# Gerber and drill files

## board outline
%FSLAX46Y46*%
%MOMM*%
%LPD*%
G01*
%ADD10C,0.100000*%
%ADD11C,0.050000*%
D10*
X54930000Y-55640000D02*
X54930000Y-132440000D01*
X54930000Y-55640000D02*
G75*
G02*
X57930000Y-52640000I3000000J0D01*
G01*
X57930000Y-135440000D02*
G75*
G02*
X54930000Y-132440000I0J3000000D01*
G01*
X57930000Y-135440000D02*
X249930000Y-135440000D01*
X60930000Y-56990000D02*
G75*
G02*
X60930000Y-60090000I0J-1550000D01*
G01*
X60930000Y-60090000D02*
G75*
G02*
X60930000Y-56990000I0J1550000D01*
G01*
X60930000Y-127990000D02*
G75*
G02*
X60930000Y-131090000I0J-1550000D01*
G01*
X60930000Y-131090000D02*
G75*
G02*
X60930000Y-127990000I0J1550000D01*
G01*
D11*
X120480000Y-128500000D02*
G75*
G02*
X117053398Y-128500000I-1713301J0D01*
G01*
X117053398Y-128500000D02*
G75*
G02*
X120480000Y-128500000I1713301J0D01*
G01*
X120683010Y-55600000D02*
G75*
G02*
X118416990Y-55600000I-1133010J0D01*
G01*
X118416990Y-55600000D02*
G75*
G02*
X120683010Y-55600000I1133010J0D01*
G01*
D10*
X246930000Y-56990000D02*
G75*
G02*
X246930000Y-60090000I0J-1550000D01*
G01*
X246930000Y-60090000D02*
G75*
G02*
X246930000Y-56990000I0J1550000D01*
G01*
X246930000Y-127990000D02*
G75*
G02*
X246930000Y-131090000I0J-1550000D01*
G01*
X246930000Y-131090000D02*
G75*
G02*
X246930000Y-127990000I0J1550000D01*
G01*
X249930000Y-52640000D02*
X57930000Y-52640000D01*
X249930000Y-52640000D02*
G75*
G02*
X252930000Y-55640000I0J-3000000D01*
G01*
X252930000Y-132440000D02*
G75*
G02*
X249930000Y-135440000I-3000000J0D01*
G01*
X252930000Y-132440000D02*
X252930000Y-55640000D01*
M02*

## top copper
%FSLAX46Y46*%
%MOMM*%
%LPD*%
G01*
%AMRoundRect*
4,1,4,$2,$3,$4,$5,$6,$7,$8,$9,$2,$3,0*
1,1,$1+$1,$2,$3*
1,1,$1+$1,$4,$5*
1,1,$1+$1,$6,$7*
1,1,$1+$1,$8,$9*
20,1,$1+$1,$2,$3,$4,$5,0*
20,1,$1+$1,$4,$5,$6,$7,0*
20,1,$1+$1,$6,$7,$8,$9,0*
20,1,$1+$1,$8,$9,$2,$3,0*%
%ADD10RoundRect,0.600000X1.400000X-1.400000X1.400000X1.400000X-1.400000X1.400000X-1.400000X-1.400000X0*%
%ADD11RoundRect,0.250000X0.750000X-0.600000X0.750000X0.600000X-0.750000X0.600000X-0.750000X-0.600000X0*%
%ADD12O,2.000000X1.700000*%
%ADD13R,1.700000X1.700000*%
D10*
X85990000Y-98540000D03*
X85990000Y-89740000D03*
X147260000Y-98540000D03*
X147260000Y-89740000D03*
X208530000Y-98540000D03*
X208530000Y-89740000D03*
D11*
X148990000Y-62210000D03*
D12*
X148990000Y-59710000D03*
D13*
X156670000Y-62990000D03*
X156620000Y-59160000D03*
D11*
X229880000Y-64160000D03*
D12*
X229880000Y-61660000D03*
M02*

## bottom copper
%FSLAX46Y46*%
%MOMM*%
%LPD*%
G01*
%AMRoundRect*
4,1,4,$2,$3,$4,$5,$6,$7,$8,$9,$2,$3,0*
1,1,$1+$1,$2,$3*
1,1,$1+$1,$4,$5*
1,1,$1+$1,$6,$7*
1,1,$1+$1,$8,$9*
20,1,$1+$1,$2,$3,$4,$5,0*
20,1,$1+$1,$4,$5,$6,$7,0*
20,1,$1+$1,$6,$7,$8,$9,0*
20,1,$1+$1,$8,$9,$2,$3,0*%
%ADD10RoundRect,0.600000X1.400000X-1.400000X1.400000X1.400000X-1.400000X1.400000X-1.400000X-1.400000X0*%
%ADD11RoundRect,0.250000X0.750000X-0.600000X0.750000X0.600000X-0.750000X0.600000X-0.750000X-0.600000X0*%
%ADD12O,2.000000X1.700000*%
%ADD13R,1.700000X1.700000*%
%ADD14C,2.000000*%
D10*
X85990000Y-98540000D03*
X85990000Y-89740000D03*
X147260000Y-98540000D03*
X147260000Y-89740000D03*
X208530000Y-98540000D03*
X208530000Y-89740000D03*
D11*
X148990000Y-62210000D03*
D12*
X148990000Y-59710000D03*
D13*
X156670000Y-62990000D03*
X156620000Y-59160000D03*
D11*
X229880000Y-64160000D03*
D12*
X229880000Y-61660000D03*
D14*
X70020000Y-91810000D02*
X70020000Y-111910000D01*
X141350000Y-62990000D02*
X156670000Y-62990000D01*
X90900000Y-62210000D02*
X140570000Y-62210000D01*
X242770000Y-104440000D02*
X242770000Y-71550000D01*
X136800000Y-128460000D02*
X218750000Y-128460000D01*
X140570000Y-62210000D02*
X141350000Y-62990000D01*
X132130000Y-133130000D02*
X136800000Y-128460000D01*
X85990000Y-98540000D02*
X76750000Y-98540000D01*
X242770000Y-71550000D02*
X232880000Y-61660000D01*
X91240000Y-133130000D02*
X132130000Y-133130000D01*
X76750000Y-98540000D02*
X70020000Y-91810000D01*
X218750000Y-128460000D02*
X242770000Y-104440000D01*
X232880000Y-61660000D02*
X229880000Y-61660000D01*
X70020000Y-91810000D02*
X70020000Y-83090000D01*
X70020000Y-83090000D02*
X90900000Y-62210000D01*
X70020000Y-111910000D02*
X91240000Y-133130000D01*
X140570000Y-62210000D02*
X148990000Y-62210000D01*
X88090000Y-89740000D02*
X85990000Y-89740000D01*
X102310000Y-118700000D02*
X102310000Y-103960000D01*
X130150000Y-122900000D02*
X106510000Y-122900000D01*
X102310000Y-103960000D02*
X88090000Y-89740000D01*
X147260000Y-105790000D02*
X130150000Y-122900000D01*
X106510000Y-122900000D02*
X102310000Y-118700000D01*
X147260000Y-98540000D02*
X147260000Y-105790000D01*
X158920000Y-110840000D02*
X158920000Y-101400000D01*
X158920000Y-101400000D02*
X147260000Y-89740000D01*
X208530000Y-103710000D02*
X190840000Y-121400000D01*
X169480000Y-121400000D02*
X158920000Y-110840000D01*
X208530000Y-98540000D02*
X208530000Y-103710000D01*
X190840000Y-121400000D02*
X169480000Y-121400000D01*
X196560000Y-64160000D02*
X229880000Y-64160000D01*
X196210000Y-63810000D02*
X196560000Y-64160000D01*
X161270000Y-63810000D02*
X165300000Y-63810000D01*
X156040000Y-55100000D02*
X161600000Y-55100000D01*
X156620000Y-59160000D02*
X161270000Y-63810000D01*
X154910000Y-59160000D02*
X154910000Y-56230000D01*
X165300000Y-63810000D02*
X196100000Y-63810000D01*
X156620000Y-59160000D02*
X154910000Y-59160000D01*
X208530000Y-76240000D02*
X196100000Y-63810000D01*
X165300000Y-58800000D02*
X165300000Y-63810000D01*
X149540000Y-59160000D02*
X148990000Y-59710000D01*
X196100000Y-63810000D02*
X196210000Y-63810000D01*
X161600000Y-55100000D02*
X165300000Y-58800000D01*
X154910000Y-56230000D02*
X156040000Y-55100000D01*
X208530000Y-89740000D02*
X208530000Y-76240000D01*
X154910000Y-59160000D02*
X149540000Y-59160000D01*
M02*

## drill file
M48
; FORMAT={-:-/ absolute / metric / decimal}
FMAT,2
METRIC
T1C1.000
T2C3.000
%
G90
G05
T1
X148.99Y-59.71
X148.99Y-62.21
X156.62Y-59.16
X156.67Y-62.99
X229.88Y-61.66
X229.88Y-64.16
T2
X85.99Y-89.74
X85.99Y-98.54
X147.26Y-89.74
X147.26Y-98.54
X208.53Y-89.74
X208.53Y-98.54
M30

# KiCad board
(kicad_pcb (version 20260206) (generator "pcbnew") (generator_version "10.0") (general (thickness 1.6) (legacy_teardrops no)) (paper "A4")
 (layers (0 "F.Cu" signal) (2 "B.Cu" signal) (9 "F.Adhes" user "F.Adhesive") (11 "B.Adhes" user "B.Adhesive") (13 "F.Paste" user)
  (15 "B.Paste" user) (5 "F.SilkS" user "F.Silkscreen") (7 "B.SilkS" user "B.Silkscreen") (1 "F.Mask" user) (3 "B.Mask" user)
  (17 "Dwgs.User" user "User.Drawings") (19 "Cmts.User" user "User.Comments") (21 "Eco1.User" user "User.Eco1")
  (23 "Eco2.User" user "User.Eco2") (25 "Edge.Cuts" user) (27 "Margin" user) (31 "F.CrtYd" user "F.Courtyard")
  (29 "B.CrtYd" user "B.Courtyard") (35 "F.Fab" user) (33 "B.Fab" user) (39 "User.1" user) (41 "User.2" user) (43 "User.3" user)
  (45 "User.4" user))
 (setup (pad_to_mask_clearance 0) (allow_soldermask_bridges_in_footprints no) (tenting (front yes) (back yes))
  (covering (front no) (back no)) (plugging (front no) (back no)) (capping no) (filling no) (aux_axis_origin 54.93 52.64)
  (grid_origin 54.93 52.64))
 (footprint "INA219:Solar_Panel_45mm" (layer "F.Cu") (at 85.99 94.14 90)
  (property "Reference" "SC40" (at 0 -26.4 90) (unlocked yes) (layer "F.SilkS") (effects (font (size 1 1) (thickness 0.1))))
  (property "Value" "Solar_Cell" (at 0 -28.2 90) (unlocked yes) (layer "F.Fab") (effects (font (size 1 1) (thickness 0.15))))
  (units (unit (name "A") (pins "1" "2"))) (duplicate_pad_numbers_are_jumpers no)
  (pad "1" thru_hole roundrect (at -4.4 0 90) (size 4 4) (drill 3) (layers "*.Cu" "*.Mask") (remove_unused_layers no)
   (roundrect_rratio 0.15) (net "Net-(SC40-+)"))
  (pad "2" thru_hole roundrect (at 4.4 0 90) (size 4 4) (drill 3) (layers "*.Cu" "*.Mask") (remove_unused_layers no) (roundrect_rratio 0.15)
   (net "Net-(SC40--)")))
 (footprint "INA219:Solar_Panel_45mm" (layer "F.Cu") (at 147.26 94.14 90)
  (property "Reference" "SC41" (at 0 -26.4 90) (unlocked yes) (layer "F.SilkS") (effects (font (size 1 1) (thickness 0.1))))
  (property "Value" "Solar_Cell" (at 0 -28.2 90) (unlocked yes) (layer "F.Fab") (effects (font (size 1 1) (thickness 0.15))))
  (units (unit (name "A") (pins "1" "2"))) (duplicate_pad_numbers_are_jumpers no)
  (pad "1" thru_hole roundrect (at -4.4 0 90) (size 4 4) (drill 3) (layers "*.Cu" "*.Mask") (remove_unused_layers no)
   (roundrect_rratio 0.15) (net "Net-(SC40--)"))
  (pad "2" thru_hole roundrect (at 4.4 0 90) (size 4 4) (drill 3) (layers "*.Cu" "*.Mask") (remove_unused_layers no) (roundrect_rratio 0.15)
   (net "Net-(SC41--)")))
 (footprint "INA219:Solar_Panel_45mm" (layer "F.Cu") (at 208.53 94.14 90)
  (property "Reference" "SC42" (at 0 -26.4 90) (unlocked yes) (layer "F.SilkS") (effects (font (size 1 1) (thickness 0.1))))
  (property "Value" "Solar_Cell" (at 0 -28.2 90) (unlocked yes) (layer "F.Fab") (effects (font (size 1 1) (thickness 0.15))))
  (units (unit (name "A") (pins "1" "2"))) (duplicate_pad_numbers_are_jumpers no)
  (pad "1" thru_hole roundrect (at -4.4 0 90) (size 4 4) (drill 3) (layers "*.Cu" "*.Mask") (remove_unused_layers no)
   (roundrect_rratio 0.15) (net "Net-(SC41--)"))
  (pad "2" thru_hole roundrect (at 4.4 0 90) (size 4 4) (drill 3) (layers "*.Cu" "*.Mask") (remove_unused_layers no) (roundrect_rratio 0.15)
   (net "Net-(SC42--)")))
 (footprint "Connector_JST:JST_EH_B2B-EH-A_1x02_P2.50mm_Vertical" (layer "B.Cu") (at 148.99 62.21 90)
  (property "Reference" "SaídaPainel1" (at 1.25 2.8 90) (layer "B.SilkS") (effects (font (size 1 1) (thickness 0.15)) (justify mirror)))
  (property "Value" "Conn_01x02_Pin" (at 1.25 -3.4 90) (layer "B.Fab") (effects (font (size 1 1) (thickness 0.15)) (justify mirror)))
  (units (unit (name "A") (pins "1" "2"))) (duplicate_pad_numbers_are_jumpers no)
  (pad "1" thru_hole roundrect (at 0 0 90) (size 1.7 2) (drill 1) (layers "*.Cu" "*.Mask") (remove_unused_layers no)
   (roundrect_rratio 0.147059) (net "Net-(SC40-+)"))
  (pad "2" thru_hole oval (at 2.5 0 90) (size 1.7 2) (drill 1) (layers "*.Cu" "*.Mask") (remove_unused_layers no) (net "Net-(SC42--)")))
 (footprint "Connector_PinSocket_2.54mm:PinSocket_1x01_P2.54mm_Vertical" (layer "B.Cu") (at 156.67 62.99 90)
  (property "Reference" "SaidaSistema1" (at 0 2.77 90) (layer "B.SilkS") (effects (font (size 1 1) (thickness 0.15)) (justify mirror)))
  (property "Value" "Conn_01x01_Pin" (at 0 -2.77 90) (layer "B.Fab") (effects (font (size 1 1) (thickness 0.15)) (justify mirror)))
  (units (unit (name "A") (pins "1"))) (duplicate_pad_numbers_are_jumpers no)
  (pad "1" thru_hole rect (at 0 0 90) (size 1.7 1.7) (drill 1) (layers "*.Cu" "*.Mask") (remove_unused_layers no) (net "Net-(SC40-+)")))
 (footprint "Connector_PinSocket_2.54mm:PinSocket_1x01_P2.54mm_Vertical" (layer "B.Cu") (at 156.62 59.16 90)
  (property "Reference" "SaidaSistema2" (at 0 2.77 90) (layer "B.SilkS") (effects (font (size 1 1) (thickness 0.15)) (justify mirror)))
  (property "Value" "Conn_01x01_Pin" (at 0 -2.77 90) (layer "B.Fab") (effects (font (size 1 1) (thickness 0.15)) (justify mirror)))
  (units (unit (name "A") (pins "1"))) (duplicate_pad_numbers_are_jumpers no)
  (pad "1" thru_hole rect (at 0 0 90) (size 1.7 1.7) (drill 1) (layers "*.Cu" "*.Mask") (remove_unused_layers no) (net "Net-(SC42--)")))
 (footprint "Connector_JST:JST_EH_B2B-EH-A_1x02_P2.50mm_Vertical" (layer "B.Cu") (at 229.88 64.16 90)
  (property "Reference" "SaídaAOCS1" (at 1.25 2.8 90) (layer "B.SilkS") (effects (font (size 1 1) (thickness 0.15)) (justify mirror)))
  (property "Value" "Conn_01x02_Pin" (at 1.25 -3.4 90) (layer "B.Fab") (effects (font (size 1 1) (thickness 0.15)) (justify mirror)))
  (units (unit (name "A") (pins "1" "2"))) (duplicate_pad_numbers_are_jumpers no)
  (pad "1" thru_hole roundrect (at 0 0 90) (size 1.7 2) (drill 1) (layers "*.Cu" "*.Mask") (remove_unused_layers no)
   (roundrect_rratio 0.147059) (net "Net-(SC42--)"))
  (pad "2" thru_hole oval (at 2.5 0 90) (size 1.7 2) (drill 1) (layers "*.Cu" "*.Mask") (remove_unused_layers no) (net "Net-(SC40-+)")))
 (gr_line (start 54.93 55.64) (end 54.93 132.44) (stroke (width 0.1) (type default)) (layer "Edge.Cuts"))
 (gr_arc (start 54.93 55.64) (mid 55.80868 53.51868) (end 57.93 52.64) (stroke (width 0.1) (type default)) (layer "Edge.Cuts"))
 (gr_arc (start 57.93 135.44) (mid 55.80868 134.56132) (end 54.93 132.44) (stroke (width 0.1) (type default)) (layer "Edge.Cuts"))
 (gr_line (start 57.93 135.44) (end 249.93 135.44) (stroke (width 0.1) (type default)) (layer "Edge.Cuts"))
 (gr_arc (start 60.93 56.99) (mid 62.48 58.54) (end 60.93 60.09) (stroke (width 0.1) (type default)) (layer "Edge.Cuts"))
 (gr_arc (start 60.93 60.09) (mid 59.38 58.54) (end 60.93 56.99) (stroke (width 0.1) (type default)) (layer "Edge.Cuts"))
 (gr_arc (start 60.93 127.99) (mid 62.48 129.54) (end 60.93 131.09) (stroke (width 0.1) (type default)) (layer "Edge.Cuts"))
 (gr_arc (start 60.93 131.09) (mid 59.38 129.54) (end 60.93 127.99) (stroke (width 0.1) (type default)) (layer "Edge.Cuts"))
 (gr_circle (center 118.766699 128.5) (end 120.316699 127.77) (stroke (width 0.05) (type default)) (fill no) (layer "Edge.Cuts"))
 (gr_circle (center 119.55 55.6) (end 120.68301 55.6) (stroke (width 0.05) (type solid)) (fill no) (layer "Edge.Cuts"))
 (gr_arc (start 246.93 56.99) (mid 248.48 58.54) (end 246.93 60.09) (stroke (width 0.1) (type default)) (layer "Edge.Cuts"))
 (gr_arc (start 246.93 60.09) (mid 245.38 58.54) (end 246.93 56.99) (stroke (width 0.1) (type default)) (layer "Edge.Cuts"))
 (gr_arc (start 246.93 127.99) (mid 248.48 129.54) (end 246.93 131.09) (stroke (width 0.1) (type default)) (layer "Edge.Cuts"))
 (gr_arc (start 246.93 131.09) (mid 245.38 129.54) (end 246.93 127.99) (stroke (width 0.1) (type default)) (layer "Edge.Cuts"))
 (gr_line (start 249.93 52.64) (end 57.93 52.64) (stroke (width 0.1) (type default)) (layer "Edge.Cuts"))
 (gr_arc (start 249.93 52.64) (mid 252.05132 53.51868) (end 252.93 55.64) (stroke (width 0.1) (type default)) (layer "Edge.Cuts"))
 (gr_arc (start 252.93 132.44) (mid 252.05132 134.56132) (end 249.93 135.44) (stroke (width 0.1) (type default)) (layer "Edge.Cuts"))
 (gr_line (start 252.93 132.44) (end 252.93 55.64) (stroke (width 0.1) (type default)) (layer "Edge.Cuts"))
 (segment (start 70.02 91.81) (end 70.02 111.91) (width 2) (layer "B.Cu") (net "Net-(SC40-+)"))
 (segment (start 141.35 62.99) (end 156.67 62.99) (width 2) (layer "B.Cu") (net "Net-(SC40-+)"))
 (segment (start 90.9 62.21) (end 140.57 62.21) (width 2) (layer "B.Cu") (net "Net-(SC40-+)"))
 (segment (start 242.77 104.44) (end 242.77 71.55) (width 2) (layer "B.Cu") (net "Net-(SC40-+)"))
 (segment (start 136.8 128.46) (end 218.75 128.46) (width 2) (layer "B.Cu") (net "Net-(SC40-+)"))
 (segment (start 140.57 62.21) (end 141.35 62.99) (width 2) (layer "B.Cu") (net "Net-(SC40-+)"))
 (segment (start 132.13 133.13) (end 136.8 128.46) (width 2) (layer "B.Cu") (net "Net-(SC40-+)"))
 (segment (start 85.99 98.54) (end 76.75 98.54) (width 2) (layer "B.Cu") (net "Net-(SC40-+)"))
 (segment (start 242.77 71.55) (end 232.88 61.66) (width 2) (layer "B.Cu") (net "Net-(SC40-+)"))
 (segment (start 91.24 133.13) (end 132.13 133.13) (width 2) (layer "B.Cu") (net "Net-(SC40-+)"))
 (segment (start 76.75 98.54) (end 70.02 91.81) (width 2) (layer "B.Cu") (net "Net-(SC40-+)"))
 (segment (start 218.75 128.46) (end 242.77 104.44) (width 2) (layer "B.Cu") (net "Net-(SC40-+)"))
 (segment (start 232.88 61.66) (end 229.88 61.66) (width 2) (layer "B.Cu") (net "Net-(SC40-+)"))
 (segment (start 70.02 91.81) (end 70.02 83.09) (width 2) (layer "B.Cu") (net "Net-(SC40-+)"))
 (segment (start 70.02 83.09) (end 90.9 62.21) (width 2) (layer "B.Cu") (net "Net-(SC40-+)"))
 (segment (start 70.02 111.91) (end 91.24 133.13) (width 2) (layer "B.Cu") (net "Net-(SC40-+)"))
 (segment (start 140.57 62.21) (end 148.99 62.21) (width 2) (layer "B.Cu") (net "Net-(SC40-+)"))
 (segment (start 88.09 89.74) (end 85.99 89.74) (width 2) (layer "B.Cu") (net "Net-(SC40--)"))
 (segment (start 102.31 118.7) (end 102.31 103.96) (width 2) (layer "B.Cu") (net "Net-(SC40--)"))
 (segment (start 130.15 122.9) (end 106.51 122.9) (width 2) (layer "B.Cu") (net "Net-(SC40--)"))
 (segment (start 102.31 103.96) (end 88.09 89.74) (width 2) (layer "B.Cu") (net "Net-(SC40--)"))
 (segment (start 147.26 105.79) (end 130.15 122.9) (width 2) (layer "B.Cu") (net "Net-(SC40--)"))
 (segment (start 106.51 122.9) (end 102.31 118.7) (width 2) (layer "B.Cu") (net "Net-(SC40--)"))
 (segment (start 147.26 98.54) (end 147.26 105.79) (width 2) (layer "B.Cu") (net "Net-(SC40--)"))
 (segment (start 158.92 110.84) (end 158.92 101.4) (width 2) (layer "B.Cu") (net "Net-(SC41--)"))
 (segment (start 158.92 101.4) (end 147.26 89.74) (width 2) (layer "B.Cu") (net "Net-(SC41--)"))
 (segment (start 208.53 103.71) (end 190.84 121.4) (width 2) (layer "B.Cu") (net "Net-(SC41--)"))
 (segment (start 169.48 121.4) (end 158.92 110.84) (width 2) (layer "B.Cu") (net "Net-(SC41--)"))
 (segment (start 208.53 98.54) (end 208.53 103.71) (width 2) (layer "B.Cu") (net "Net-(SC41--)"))
 (segment (start 190.84 121.4) (end 169.48 121.4) (width 2) (layer "B.Cu") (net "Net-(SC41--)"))
 (segment (start 196.56 64.16) (end 229.88 64.16) (width 2) (layer "B.Cu") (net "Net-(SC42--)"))
 (segment (start 196.21 63.81) (end 196.56 64.16) (width 2) (layer "B.Cu") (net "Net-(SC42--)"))
 (segment (start 161.27 63.81) (end 165.3 63.81) (width 2) (layer "B.Cu") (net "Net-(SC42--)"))
 (segment (start 156.04 55.1) (end 161.6 55.1) (width 2) (layer "B.Cu") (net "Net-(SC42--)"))
 (segment (start 156.62 59.16) (end 161.27 63.81) (width 2) (layer "B.Cu") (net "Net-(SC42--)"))
 (segment (start 154.91 59.16) (end 154.91 56.23) (width 2) (layer "B.Cu") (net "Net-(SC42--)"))
 (segment (start 165.3 63.81) (end 196.1 63.81) (width 2) (layer "B.Cu") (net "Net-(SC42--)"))
 (segment (start 156.62 59.16) (end 154.91 59.16) (width 2) (layer "B.Cu") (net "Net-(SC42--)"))
 (segment (start 208.53 76.24) (end 196.1 63.81) (width 2) (layer "B.Cu") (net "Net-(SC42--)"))
 (segment (start 165.3 58.8) (end 165.3 63.81) (width 2) (layer "B.Cu") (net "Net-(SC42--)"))
 (segment (start 149.54 59.16) (end 148.99 59.71) (width 2) (layer "B.Cu") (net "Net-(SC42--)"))
 (segment (start 196.1 63.81) (end 196.21 63.81) (width 2) (layer "B.Cu") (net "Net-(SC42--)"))
 (segment (start 161.6 55.1) (end 165.3 58.8) (width 2) (layer "B.Cu") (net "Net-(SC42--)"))
 (segment (start 154.91 56.23) (end 156.04 55.1) (width 2) (layer "B.Cu") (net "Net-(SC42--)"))
 (segment (start 208.53 89.74) (end 208.53 76.24) (width 2) (layer "B.Cu") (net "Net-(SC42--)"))
 (segment (start 154.91 59.16) (end 149.54 59.16) (width 2) (layer "B.Cu") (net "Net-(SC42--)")))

